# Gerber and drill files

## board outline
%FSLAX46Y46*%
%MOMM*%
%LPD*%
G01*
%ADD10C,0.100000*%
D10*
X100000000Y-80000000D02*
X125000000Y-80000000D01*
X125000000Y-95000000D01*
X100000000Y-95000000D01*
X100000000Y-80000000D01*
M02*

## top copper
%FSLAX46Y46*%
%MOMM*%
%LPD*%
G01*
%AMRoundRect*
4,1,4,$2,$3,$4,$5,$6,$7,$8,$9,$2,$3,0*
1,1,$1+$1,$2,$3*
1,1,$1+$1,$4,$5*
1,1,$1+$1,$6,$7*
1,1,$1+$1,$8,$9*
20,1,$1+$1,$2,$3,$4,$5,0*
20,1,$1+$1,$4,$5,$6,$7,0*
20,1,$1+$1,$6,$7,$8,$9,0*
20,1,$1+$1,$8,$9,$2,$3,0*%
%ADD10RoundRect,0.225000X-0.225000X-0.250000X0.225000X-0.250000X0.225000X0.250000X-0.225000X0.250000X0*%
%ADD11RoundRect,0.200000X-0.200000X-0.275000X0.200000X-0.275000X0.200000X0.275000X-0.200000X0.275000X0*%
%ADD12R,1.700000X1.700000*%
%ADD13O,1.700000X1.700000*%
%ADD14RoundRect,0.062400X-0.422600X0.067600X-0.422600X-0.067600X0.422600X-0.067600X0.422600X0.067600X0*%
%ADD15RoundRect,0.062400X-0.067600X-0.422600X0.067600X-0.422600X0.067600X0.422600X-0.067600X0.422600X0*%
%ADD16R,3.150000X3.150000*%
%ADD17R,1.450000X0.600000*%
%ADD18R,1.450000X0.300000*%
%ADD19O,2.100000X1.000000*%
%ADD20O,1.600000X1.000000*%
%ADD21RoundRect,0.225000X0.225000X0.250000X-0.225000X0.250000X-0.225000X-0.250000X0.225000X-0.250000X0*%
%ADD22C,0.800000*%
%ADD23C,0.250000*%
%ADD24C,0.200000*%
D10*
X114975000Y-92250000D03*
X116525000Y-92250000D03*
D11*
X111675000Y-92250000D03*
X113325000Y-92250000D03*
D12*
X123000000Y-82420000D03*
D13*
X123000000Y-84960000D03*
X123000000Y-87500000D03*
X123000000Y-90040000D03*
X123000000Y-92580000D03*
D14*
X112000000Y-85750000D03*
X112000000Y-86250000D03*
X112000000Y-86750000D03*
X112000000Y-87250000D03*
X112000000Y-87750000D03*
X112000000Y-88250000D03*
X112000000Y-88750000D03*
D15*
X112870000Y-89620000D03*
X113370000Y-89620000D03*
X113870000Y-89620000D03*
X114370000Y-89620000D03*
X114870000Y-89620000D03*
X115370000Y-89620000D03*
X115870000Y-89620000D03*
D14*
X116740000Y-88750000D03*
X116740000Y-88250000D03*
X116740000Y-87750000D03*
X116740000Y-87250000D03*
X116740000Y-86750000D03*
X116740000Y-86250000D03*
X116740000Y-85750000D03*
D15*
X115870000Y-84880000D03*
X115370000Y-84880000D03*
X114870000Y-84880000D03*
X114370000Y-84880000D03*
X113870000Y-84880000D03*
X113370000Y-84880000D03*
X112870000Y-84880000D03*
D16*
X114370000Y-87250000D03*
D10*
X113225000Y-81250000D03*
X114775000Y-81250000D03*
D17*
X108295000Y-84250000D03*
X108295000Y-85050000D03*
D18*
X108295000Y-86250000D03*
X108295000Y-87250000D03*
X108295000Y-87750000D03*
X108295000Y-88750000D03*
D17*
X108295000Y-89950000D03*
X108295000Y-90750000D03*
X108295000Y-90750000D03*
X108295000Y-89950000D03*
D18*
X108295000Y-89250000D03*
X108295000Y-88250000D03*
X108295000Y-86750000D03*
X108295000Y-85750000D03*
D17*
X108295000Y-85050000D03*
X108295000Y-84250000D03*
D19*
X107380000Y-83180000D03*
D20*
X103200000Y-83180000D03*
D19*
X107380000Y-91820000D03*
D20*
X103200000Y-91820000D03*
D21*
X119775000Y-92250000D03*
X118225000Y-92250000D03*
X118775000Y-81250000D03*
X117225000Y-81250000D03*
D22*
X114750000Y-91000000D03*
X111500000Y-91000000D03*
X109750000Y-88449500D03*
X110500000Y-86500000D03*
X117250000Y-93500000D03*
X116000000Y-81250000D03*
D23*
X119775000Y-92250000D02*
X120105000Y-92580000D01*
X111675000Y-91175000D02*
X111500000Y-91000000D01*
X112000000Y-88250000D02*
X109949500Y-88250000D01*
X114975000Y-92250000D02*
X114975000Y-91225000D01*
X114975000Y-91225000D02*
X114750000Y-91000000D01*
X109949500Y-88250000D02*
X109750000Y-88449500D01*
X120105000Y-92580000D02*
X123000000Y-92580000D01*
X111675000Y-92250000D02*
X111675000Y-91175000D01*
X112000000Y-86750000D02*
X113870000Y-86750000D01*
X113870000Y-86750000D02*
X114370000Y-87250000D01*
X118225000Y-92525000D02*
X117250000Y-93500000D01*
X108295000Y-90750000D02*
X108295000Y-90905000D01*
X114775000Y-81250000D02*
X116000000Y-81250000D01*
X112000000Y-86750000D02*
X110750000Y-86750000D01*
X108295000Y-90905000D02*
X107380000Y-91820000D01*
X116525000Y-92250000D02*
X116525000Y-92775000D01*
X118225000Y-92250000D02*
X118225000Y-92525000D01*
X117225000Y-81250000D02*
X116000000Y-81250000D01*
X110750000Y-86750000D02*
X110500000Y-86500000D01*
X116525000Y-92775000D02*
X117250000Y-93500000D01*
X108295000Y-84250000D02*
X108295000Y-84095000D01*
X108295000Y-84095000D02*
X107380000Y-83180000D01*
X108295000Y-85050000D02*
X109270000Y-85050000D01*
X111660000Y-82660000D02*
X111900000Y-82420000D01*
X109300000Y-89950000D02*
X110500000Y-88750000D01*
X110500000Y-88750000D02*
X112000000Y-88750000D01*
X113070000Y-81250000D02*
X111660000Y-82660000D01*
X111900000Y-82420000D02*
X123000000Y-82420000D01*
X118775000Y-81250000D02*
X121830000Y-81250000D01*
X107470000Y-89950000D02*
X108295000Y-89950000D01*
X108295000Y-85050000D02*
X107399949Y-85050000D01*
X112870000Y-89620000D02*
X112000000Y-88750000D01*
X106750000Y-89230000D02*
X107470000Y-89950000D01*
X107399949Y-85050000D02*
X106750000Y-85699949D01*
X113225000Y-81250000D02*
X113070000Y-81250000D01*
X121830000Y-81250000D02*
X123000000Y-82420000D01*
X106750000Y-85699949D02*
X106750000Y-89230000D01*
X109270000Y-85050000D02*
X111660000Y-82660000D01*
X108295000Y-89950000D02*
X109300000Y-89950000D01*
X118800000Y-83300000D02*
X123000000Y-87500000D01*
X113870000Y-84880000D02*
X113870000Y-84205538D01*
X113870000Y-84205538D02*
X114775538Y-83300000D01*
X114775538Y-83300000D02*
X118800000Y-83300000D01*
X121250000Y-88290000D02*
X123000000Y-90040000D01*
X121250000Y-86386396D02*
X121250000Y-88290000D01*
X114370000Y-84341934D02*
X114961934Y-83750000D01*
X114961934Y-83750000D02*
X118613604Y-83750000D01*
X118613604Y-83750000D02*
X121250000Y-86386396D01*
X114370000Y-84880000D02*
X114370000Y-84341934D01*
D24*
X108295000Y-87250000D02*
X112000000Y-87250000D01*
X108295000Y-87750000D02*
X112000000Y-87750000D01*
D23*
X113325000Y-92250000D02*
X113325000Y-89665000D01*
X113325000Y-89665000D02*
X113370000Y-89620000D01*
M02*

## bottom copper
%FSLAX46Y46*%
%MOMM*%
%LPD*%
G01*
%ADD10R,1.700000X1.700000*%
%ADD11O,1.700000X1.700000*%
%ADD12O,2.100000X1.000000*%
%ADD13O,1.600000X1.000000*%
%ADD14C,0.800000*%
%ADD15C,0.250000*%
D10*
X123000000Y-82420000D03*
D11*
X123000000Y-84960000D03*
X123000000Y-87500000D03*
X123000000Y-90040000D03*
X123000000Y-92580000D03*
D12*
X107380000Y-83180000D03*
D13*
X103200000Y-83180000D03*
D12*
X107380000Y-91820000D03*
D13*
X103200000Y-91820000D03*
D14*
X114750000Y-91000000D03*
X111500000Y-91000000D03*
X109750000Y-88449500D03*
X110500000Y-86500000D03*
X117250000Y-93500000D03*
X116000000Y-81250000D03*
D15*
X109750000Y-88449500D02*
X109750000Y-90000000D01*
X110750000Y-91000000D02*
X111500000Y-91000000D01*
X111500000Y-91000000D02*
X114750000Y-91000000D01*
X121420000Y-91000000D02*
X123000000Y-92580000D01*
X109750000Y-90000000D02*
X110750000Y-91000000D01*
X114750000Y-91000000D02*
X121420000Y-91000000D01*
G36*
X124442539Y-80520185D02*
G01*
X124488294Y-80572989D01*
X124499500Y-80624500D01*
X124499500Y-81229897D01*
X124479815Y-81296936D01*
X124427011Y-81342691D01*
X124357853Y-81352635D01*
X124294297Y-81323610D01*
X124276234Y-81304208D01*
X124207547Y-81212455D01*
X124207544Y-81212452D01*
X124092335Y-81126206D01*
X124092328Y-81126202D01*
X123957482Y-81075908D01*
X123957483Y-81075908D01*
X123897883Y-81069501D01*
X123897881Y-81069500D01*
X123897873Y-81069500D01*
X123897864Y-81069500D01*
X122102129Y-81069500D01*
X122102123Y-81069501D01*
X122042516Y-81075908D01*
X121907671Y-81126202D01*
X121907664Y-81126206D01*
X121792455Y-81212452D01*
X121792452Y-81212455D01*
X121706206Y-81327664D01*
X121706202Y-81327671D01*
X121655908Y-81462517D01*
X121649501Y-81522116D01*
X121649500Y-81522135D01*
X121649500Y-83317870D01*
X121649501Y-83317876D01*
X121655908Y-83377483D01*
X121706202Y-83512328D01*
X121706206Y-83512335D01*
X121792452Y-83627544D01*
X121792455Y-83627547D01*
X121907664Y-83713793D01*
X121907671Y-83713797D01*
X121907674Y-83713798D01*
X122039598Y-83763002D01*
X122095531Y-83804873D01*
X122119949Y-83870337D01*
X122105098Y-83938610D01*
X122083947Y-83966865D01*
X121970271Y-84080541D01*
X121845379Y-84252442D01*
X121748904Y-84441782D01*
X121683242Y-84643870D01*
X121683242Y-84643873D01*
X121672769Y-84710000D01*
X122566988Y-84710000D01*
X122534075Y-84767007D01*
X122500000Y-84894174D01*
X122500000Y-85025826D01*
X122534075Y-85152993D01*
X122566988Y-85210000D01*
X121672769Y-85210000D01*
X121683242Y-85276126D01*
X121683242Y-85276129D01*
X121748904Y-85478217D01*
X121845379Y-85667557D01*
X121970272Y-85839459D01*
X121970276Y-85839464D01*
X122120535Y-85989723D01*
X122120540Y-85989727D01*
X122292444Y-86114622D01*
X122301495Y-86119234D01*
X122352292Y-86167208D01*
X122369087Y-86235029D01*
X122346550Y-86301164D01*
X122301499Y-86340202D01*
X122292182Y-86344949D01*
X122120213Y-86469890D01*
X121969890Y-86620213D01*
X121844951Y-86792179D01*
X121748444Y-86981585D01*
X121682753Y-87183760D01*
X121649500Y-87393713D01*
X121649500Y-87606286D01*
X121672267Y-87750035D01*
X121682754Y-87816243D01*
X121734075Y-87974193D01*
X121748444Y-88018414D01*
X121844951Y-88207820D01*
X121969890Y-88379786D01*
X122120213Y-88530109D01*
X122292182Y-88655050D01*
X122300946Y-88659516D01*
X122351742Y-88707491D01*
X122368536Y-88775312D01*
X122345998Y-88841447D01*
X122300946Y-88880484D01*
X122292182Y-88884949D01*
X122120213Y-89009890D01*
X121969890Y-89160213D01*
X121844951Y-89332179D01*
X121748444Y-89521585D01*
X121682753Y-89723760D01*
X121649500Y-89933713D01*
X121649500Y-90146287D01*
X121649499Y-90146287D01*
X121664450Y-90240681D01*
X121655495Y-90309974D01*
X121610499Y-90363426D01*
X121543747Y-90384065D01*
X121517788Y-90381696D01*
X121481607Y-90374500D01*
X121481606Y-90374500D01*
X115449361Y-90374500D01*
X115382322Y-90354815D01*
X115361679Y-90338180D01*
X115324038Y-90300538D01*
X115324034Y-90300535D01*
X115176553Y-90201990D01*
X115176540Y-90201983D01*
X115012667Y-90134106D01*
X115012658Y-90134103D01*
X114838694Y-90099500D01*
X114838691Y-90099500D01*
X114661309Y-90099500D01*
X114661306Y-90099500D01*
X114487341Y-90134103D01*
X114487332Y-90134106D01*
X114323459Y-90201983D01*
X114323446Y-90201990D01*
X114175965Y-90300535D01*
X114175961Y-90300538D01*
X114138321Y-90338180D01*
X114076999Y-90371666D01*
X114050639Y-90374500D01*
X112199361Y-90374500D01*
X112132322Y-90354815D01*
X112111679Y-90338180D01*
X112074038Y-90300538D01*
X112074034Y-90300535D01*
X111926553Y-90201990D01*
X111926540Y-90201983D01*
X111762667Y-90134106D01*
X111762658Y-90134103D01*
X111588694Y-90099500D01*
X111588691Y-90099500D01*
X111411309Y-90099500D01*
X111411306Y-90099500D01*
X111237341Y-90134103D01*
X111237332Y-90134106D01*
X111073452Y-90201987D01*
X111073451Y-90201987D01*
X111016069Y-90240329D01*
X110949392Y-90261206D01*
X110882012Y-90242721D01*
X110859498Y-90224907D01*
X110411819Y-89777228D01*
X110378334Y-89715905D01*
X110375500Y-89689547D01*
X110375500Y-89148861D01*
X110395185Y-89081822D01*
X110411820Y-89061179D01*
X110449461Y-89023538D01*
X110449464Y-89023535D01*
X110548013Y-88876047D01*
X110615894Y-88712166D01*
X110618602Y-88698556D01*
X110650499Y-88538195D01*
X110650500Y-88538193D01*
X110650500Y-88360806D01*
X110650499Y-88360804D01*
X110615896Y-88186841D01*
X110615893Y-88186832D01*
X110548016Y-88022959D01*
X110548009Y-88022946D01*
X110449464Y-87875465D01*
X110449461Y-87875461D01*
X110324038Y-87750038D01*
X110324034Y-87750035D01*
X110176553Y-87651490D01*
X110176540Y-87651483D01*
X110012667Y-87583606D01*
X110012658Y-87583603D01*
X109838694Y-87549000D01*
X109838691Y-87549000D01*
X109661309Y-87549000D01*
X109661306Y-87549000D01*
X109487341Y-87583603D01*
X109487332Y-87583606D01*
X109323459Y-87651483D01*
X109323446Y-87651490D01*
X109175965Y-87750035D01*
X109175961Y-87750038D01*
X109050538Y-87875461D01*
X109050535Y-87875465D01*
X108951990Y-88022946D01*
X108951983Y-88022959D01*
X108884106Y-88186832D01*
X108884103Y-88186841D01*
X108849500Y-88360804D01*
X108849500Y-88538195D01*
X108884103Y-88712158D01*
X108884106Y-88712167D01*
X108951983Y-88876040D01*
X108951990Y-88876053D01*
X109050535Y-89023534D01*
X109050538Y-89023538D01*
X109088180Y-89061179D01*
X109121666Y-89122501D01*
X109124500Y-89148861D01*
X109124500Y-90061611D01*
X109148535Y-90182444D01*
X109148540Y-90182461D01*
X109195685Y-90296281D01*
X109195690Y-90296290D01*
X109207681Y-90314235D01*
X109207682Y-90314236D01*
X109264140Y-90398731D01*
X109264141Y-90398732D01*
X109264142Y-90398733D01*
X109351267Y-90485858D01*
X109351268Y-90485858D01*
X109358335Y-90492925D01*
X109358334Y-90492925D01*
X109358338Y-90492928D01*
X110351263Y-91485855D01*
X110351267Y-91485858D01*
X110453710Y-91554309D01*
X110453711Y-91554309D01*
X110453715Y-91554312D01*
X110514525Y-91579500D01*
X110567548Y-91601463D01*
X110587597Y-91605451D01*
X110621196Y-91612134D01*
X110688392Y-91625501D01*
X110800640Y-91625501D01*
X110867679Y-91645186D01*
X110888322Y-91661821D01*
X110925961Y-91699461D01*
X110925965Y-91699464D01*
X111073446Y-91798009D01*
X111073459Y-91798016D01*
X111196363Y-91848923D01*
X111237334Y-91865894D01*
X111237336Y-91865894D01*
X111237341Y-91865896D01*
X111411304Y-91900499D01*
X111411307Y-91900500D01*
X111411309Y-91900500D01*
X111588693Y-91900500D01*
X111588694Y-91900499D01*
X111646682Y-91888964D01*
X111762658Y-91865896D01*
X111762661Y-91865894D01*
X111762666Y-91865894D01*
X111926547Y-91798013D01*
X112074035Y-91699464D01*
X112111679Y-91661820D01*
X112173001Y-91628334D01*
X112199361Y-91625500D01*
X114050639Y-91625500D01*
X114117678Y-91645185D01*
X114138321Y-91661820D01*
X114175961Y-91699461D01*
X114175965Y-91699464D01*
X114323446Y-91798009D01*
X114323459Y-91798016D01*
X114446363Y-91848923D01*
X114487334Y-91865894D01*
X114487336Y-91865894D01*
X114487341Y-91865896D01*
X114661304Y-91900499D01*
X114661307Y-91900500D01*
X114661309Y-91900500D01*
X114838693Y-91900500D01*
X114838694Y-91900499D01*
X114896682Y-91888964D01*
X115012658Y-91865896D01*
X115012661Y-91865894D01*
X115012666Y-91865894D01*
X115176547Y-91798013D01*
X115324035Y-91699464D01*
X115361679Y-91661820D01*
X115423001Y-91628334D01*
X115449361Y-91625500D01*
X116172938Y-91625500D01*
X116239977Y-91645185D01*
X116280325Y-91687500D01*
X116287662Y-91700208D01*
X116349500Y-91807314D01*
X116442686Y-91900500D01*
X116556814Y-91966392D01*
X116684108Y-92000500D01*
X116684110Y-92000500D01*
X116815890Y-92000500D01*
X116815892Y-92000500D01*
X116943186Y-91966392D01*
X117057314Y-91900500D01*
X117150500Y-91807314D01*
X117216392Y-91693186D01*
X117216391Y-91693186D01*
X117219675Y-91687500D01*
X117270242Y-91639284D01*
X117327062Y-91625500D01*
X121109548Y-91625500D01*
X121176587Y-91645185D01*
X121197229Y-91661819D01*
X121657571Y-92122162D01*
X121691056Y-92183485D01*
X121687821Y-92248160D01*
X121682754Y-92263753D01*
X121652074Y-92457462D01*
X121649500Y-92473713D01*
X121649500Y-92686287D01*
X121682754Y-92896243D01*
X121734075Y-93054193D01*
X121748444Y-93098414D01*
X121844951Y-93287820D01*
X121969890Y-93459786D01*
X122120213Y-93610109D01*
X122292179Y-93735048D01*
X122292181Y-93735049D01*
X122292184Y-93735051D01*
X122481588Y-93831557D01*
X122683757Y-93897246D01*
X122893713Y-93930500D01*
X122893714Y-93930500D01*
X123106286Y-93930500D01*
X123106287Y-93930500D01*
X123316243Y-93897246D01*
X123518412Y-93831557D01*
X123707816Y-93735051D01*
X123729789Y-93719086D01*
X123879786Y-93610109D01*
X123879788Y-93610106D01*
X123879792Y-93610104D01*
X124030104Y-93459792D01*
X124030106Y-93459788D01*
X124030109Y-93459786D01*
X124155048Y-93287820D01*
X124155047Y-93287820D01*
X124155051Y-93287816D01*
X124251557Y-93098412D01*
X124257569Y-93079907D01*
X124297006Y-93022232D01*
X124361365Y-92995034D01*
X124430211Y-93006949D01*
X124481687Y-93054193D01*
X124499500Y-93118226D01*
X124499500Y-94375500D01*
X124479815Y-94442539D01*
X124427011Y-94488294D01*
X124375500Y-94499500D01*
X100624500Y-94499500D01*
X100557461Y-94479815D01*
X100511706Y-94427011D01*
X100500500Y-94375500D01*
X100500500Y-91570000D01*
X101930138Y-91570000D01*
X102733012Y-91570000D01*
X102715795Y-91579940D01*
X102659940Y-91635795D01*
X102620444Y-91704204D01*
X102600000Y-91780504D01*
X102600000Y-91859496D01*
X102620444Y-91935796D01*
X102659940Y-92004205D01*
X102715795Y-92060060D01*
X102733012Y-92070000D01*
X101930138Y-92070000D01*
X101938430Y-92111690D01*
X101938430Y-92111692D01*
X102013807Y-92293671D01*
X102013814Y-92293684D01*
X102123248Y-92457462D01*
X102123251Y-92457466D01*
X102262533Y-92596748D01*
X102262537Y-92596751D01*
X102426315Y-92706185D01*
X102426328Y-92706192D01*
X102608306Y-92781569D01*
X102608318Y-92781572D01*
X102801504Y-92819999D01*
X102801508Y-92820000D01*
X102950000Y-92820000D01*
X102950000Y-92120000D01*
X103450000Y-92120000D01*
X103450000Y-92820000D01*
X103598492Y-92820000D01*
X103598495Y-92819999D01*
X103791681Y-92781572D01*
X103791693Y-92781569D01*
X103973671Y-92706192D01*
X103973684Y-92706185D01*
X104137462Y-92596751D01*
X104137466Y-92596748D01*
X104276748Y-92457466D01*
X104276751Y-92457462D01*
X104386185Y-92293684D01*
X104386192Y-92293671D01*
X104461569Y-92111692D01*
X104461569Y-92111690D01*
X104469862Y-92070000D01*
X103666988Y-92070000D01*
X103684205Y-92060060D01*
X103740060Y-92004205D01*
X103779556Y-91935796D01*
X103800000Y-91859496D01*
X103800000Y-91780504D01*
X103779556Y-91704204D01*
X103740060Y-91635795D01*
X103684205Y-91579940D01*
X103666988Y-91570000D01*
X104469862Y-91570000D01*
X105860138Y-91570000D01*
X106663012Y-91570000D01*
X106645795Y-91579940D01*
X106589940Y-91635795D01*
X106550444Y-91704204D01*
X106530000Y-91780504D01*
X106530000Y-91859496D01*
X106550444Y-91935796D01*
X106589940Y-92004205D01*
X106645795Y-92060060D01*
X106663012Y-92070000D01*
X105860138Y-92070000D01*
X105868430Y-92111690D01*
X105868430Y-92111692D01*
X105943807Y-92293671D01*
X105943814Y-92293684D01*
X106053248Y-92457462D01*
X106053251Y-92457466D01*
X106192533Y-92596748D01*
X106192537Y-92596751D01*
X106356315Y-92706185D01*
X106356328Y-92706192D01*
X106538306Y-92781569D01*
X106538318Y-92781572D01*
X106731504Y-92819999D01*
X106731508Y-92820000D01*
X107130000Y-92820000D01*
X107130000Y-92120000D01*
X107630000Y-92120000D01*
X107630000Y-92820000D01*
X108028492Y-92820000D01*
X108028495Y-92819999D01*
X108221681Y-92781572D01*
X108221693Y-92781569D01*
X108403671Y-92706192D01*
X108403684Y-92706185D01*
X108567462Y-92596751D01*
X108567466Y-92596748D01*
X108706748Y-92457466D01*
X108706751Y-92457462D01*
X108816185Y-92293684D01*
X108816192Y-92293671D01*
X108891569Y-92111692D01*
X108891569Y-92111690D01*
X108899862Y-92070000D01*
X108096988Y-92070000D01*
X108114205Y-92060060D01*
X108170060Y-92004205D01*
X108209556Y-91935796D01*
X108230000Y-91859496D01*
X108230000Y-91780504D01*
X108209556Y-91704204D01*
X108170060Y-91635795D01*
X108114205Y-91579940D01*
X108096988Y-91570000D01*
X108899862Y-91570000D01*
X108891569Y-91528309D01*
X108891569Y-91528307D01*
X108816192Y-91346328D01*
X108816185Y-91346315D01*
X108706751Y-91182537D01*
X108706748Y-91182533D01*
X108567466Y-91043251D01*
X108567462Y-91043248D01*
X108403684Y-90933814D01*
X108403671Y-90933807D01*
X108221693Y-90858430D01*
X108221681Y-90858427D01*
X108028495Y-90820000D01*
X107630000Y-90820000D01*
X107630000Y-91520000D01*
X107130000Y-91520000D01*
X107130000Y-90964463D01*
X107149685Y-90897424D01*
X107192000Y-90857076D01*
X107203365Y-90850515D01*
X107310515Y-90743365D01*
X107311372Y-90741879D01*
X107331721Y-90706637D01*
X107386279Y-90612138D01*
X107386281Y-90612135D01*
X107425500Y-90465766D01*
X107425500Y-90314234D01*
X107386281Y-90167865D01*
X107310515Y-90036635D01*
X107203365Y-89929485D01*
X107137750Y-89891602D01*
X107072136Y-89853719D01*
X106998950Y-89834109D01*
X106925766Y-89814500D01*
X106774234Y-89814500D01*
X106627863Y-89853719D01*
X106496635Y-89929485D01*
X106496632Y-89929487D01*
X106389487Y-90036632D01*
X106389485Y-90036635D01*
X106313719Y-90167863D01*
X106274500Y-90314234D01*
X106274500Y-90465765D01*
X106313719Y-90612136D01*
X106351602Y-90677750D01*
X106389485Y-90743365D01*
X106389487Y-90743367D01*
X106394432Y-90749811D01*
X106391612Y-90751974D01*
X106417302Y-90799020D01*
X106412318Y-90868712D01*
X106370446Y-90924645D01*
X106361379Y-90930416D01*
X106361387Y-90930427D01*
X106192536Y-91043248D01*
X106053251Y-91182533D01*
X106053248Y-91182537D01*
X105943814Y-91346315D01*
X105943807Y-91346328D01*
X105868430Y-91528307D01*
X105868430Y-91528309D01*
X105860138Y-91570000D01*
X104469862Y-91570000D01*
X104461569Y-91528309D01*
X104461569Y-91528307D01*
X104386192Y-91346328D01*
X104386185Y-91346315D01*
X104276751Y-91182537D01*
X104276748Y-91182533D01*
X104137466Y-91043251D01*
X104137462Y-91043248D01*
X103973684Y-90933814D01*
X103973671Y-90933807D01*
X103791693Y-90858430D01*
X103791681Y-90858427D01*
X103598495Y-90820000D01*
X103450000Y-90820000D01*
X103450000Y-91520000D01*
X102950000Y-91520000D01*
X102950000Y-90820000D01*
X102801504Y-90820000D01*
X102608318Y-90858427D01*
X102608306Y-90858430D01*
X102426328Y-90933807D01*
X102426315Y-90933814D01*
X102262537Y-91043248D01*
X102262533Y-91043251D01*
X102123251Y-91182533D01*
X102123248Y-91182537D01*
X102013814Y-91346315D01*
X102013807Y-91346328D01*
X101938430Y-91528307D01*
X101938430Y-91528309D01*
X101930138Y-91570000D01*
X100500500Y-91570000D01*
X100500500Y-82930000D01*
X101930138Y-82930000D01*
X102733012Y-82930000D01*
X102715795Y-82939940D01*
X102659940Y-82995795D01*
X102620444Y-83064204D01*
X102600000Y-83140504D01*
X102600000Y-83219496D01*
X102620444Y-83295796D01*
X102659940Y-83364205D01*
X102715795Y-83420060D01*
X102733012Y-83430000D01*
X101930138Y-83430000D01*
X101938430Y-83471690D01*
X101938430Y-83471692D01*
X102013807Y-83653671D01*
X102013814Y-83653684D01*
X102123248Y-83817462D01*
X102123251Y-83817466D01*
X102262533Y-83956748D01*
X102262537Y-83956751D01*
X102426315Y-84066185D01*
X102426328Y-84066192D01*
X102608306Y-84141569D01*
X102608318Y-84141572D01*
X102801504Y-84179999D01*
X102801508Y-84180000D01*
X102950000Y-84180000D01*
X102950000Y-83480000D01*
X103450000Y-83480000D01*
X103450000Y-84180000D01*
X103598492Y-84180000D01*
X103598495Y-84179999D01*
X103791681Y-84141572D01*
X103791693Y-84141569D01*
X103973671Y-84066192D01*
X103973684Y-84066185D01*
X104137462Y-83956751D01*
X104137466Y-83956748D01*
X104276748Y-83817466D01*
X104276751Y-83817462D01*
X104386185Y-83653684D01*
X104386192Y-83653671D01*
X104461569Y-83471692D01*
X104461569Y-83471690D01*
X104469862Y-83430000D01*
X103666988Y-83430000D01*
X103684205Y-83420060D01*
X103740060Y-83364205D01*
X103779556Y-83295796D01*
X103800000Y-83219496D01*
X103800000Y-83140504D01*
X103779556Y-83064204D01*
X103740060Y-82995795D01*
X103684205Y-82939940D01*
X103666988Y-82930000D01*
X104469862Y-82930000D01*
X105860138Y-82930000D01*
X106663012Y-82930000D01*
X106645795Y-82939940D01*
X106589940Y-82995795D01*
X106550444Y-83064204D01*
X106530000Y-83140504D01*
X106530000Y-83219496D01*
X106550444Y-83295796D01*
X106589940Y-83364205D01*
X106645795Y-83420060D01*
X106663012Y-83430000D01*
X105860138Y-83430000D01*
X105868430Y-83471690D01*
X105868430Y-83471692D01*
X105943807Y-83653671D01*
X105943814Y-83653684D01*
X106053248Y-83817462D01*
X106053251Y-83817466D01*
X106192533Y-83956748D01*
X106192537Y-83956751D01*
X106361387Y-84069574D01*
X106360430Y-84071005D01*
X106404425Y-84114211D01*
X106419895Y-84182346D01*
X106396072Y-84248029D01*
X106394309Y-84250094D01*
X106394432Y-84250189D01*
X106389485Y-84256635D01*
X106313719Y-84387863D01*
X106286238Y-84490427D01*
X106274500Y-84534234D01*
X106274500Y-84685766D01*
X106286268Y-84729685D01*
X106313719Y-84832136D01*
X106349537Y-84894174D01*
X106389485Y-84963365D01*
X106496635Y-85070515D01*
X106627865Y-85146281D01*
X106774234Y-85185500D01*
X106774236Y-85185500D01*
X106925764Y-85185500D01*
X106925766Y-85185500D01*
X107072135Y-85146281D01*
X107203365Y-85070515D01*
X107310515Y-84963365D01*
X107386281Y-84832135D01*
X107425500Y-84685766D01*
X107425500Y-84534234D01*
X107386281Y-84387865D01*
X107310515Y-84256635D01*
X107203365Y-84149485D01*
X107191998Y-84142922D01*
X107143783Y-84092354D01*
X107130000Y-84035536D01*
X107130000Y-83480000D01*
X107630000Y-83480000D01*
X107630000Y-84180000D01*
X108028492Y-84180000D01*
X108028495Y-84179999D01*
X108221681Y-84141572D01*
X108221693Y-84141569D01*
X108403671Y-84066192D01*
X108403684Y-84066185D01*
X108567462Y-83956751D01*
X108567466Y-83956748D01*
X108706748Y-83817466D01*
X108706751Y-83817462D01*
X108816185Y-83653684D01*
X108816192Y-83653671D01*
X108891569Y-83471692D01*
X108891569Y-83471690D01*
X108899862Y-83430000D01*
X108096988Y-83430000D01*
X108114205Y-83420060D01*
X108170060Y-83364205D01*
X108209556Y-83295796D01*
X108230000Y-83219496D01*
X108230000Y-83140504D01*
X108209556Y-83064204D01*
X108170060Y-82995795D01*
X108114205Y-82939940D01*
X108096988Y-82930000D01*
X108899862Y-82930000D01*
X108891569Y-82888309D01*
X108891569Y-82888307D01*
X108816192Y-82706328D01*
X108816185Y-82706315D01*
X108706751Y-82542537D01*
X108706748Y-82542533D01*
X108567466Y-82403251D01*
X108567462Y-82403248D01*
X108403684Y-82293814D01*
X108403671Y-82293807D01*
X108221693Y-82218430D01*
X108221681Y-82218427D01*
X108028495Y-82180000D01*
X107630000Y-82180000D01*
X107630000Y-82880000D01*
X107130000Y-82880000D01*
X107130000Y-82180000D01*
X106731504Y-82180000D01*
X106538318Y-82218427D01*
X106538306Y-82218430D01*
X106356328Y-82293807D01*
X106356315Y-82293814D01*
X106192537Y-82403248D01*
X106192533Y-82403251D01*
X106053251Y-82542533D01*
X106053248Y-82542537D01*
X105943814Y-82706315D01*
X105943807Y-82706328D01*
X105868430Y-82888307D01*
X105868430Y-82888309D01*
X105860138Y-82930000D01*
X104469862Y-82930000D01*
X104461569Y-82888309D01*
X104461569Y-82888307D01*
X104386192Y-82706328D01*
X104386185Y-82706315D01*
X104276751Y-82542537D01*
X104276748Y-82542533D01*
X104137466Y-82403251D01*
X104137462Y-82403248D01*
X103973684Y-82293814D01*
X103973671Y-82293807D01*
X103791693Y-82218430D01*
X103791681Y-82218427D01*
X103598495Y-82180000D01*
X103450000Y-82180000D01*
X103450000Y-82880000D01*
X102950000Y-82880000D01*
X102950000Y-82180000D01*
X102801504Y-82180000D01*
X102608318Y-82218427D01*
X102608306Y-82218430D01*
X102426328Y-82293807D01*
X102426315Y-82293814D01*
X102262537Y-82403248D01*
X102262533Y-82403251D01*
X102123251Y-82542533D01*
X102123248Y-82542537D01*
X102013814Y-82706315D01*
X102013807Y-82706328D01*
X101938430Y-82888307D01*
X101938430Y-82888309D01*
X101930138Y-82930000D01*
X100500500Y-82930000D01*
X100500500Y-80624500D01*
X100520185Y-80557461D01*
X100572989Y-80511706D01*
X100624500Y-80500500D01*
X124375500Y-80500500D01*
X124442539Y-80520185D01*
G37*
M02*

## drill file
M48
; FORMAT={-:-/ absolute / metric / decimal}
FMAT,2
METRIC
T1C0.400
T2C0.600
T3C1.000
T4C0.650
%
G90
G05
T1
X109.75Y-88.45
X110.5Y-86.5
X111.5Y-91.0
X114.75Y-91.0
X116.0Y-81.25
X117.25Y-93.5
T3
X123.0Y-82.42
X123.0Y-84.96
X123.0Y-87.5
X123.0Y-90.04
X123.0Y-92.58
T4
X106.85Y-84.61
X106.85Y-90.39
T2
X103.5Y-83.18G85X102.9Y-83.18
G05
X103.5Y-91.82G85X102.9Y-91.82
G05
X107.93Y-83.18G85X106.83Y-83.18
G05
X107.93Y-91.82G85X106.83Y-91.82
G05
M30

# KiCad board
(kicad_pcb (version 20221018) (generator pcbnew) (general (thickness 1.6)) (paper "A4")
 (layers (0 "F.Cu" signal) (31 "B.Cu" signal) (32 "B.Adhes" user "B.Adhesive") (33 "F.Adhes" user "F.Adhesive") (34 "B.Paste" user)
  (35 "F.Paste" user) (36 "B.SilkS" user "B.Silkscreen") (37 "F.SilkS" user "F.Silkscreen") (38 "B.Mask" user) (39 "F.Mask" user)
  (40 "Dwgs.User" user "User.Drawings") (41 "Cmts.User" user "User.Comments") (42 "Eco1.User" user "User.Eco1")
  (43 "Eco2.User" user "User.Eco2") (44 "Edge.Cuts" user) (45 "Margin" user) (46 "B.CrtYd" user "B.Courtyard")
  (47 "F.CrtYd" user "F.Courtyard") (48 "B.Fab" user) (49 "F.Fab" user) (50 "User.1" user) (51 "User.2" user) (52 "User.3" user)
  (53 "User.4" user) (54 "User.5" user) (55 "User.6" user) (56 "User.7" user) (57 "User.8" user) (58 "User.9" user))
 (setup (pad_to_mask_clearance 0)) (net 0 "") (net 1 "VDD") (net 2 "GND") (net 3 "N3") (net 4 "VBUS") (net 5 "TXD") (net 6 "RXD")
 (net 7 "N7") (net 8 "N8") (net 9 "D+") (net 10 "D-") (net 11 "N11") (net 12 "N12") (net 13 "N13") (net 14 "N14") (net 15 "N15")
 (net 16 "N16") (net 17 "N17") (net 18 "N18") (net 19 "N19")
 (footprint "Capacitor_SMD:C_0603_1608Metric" (layer "F.Cu") (at 115.75 92.25)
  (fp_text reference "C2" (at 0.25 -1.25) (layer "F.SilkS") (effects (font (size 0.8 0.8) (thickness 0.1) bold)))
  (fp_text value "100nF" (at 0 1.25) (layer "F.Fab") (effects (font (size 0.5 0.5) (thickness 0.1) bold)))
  (pad "1" smd roundrect (at -0.775 0) (size 0.9 0.95) (layers "F.Cu" "F.Paste" "F.Mask") (roundrect_rratio 0.25) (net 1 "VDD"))
  (pad "2" smd roundrect (at 0.775 0) (size 0.9 0.95) (layers "F.Cu" "F.Paste" "F.Mask") (roundrect_rratio 0.25) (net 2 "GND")))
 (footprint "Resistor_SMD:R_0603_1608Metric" (layer "F.Cu") (at 112.5 92.25)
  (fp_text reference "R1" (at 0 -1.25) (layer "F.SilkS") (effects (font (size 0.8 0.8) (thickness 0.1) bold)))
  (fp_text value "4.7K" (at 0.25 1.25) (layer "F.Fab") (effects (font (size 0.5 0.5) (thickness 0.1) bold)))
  (pad "1" smd roundrect (at -0.825 0) (size 0.8 0.95) (layers "F.Cu" "F.Paste" "F.Mask") (roundrect_rratio 0.25) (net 1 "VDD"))
  (pad "2" smd roundrect (at 0.825 0) (size 0.8 0.95) (layers "F.Cu" "F.Paste" "F.Mask") (roundrect_rratio 0.25) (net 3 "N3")))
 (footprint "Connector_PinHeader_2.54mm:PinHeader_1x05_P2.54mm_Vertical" (layer "F.Cu") (at 123 82.42)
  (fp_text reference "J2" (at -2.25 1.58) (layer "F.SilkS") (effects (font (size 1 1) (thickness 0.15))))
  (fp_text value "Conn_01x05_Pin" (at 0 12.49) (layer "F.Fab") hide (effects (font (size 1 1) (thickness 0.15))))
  (pad "1" thru_hole rect (at 0 0) (size 1.7 1.7) (drill 1) (layers "*.Cu" "*.Mask") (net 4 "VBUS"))
  (pad "2" thru_hole oval (at 0 2.54) (size 1.7 1.7) (drill 1) (layers "*.Cu" "*.Mask") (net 2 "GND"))
  (pad "3" thru_hole oval (at 0 5.08) (size 1.7 1.7) (drill 1) (layers "*.Cu" "*.Mask") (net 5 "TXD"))
  (pad "4" thru_hole oval (at 0 7.62) (size 1.7 1.7) (drill 1) (layers "*.Cu" "*.Mask") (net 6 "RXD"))
  (pad "5" thru_hole oval (at 0 10.16) (size 1.7 1.7) (drill 1) (layers "*.Cu" "*.Mask") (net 1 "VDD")))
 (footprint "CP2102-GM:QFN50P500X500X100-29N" (layer "F.Cu") (at 114.37 87.25)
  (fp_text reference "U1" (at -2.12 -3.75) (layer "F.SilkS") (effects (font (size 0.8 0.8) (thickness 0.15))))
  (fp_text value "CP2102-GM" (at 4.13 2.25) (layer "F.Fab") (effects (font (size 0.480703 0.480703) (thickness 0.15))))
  (pad "1" smd roundrect (at -2.37 -1.5 270) (size 0.26 0.97) (layers "F.Cu" "F.Paste" "F.Mask") (roundrect_rratio 0.24) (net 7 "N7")
   (solder_mask_margin 0.102))
  (pad "2" smd roundrect (at -2.37 -1 270) (size 0.26 0.97) (layers "F.Cu" "F.Paste" "F.Mask") (roundrect_rratio 0.24) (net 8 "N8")
   (solder_mask_margin 0.102))
  (pad "3" smd roundrect (at -2.37 -0.5 270) (size 0.26 0.97) (layers "F.Cu" "F.Paste" "F.Mask") (roundrect_rratio 0.24) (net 2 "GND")
   (solder_mask_margin 0.102))
  (pad "4" smd roundrect (at -2.37 0 270) (size 0.26 0.97) (layers "F.Cu" "F.Paste" "F.Mask") (roundrect_rratio 0.24) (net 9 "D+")
   (solder_mask_margin 0.102))
  (pad "5" smd roundrect (at -2.37 0.5 270) (size 0.26 0.97) (layers "F.Cu" "F.Paste" "F.Mask") (roundrect_rratio 0.24) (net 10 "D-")
   (solder_mask_margin 0.102))
  (pad "6" smd roundrect (at -2.37 1 270) (size 0.26 0.97) (layers "F.Cu" "F.Paste" "F.Mask") (roundrect_rratio 0.24) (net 1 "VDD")
   (solder_mask_margin 0.102))
  (pad "7" smd roundrect (at -2.37 1.5 270) (size 0.26 0.97) (layers "F.Cu" "F.Paste" "F.Mask") (roundrect_rratio 0.24) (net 4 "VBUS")
   (solder_mask_margin 0.102))
  (pad "8" smd roundrect (at -1.5 2.37) (size 0.26 0.97) (layers "F.Cu" "F.Paste" "F.Mask") (roundrect_rratio 0.24) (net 4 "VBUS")
   (solder_mask_margin 0.102))
  (pad "9" smd roundrect (at -1 2.37) (size 0.26 0.97) (layers "F.Cu" "F.Paste" "F.Mask") (roundrect_rratio 0.24) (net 3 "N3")
   (solder_mask_margin 0.102))
  (pad "10" smd roundrect (at -0.5 2.37) (size 0.26 0.97) (layers "F.Cu" "F.Paste" "F.Mask") (roundrect_rratio 0.24)
   (solder_mask_margin 0.102))
  (pad "11" smd roundrect (at 0 2.37) (size 0.26 0.97) (layers "F.Cu" "F.Paste" "F.Mask") (roundrect_rratio 0.24) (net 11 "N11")
   (solder_mask_margin 0.102))
  (pad "12" smd roundrect (at 0.5 2.37) (size 0.26 0.97) (layers "F.Cu" "F.Paste" "F.Mask") (roundrect_rratio 0.24) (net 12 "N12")
   (solder_mask_margin 0.102))
  (pad "13" smd roundrect (at 1 2.37) (size 0.26 0.97) (layers "F.Cu" "F.Paste" "F.Mask") (roundrect_rratio 0.24) (solder_mask_margin 0.102))
  (pad "14" smd roundrect (at 1.5 2.37) (size 0.26 0.97) (layers "F.Cu" "F.Paste" "F.Mask") (roundrect_rratio 0.24)
   (solder_mask_margin 0.102))
  (pad "15" smd roundrect (at 2.37 1.5 270) (size 0.26 0.97) (layers "F.Cu" "F.Paste" "F.Mask") (roundrect_rratio 0.24)
   (solder_mask_margin 0.102))
  (pad "16" smd roundrect (at 2.37 1 270) (size 0.26 0.97) (layers "F.Cu" "F.Paste" "F.Mask") (roundrect_rratio 0.24)
   (solder_mask_margin 0.102))
  (pad "17" smd roundrect (at 2.37 0.5 270) (size 0.26 0.97) (layers "F.Cu" "F.Paste" "F.Mask") (roundrect_rratio 0.24)
   (solder_mask_margin 0.102))
  (pad "18" smd roundrect (at 2.37 0 270) (size 0.26 0.97) (layers "F.Cu" "F.Paste" "F.Mask") (roundrect_rratio 0.24) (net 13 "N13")
   (solder_mask_margin 0.102))
  (pad "19" smd roundrect (at 2.37 -0.5 270) (size 0.26 0.97) (layers "F.Cu" "F.Paste" "F.Mask") (roundrect_rratio 0.24)
   (solder_mask_margin 0.102))
  (pad "20" smd roundrect (at 2.37 -1 270) (size 0.26 0.97) (layers "F.Cu" "F.Paste" "F.Mask") (roundrect_rratio 0.24)
   (solder_mask_margin 0.102))
  (pad "21" smd roundrect (at 2.37 -1.5 270) (size 0.26 0.97) (layers "F.Cu" "F.Paste" "F.Mask") (roundrect_rratio 0.24)
   (solder_mask_margin 0.102))
  (pad "22" smd roundrect (at 1.5 -2.37) (size 0.26 0.97) (layers "F.Cu" "F.Paste" "F.Mask") (roundrect_rratio 0.24)
   (solder_mask_margin 0.102))
  (pad "23" smd roundrect (at 1 -2.37) (size 0.26 0.97) (layers "F.Cu" "F.Paste" "F.Mask") (roundrect_rratio 0.24) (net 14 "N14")
   (solder_mask_margin 0.102))
  (pad "24" smd roundrect (at 0.5 -2.37) (size 0.26 0.97) (layers "F.Cu" "F.Paste" "F.Mask") (roundrect_rratio 0.24) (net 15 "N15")
   (solder_mask_margin 0.102))
  (pad "25" smd roundrect (at 0 -2.37) (size 0.26 0.97) (layers "F.Cu" "F.Paste" "F.Mask") (roundrect_rratio 0.24) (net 6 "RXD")
   (solder_mask_margin 0.102))
  (pad "26" smd roundrect (at -0.5 -2.37) (size 0.26 0.97) (layers "F.Cu" "F.Paste" "F.Mask") (roundrect_rratio 0.24) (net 5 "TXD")
   (solder_mask_margin 0.102))
  (pad "27" smd roundrect (at -1 -2.37) (size 0.26 0.97) (layers "F.Cu" "F.Paste" "F.Mask") (roundrect_rratio 0.24) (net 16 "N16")
   (solder_mask_margin 0.102))
  (pad "28" smd roundrect (at -1.5 -2.37) (size 0.26 0.97) (layers "F.Cu" "F.Paste" "F.Mask") (roundrect_rratio 0.24) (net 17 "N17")
   (solder_mask_margin 0.102))
  (pad "29" smd rect (at 0 0) (size 3.15 3.15) (layers "F.Cu" "F.Mask") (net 2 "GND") (solder_mask_margin 0.102)))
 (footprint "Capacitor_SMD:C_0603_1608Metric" (layer "F.Cu") (at 114 81.25)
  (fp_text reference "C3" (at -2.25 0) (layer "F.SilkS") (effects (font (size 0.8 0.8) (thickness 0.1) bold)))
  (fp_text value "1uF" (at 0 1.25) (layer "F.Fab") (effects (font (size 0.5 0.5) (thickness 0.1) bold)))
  (pad "1" smd roundrect (at -0.775 0) (size 0.9 0.95) (layers "F.Cu" "F.Paste" "F.Mask") (roundrect_rratio 0.25) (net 4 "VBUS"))
  (pad "2" smd roundrect (at 0.775 0) (size 0.9 0.95) (layers "F.Cu" "F.Paste" "F.Mask") (roundrect_rratio 0.25) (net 2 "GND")))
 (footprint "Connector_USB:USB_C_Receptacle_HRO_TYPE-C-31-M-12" (layer "F.Cu") (at 104.25 87.5 -90)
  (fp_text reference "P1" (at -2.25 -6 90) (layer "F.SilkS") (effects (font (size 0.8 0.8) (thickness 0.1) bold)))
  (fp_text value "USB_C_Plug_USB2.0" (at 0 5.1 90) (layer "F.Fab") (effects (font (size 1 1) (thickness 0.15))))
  (pad "" np_thru_hole circle (at -2.89 -2.6 270) (size 0.65 0.65) (drill 0.65) (layers "*.Cu" "*.Mask"))
  (pad "" np_thru_hole circle (at 2.89 -2.6 270) (size 0.65 0.65) (drill 0.65) (layers "*.Cu" "*.Mask"))
  (pad "A1" smd rect (at -3.25 -4.045 270) (size 0.6 1.45) (layers "F.Cu" "F.Paste" "F.Mask") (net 2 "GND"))
  (pad "A4" smd rect (at -2.45 -4.045 270) (size 0.6 1.45) (layers "F.Cu" "F.Paste" "F.Mask") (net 4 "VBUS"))
  (pad "A5" smd rect (at -1.25 -4.045 270) (size 0.3 1.45) (layers "F.Cu" "F.Paste" "F.Mask") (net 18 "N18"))
  (pad "A6" smd rect (at -0.25 -4.045 270) (size 0.3 1.45) (layers "F.Cu" "F.Paste" "F.Mask") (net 9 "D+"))
  (pad "A7" smd rect (at 0.25 -4.045 270) (size 0.3 1.45) (layers "F.Cu" "F.Paste" "F.Mask") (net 10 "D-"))
  (pad "A8" smd rect (at 1.25 -4.045 270) (size 0.3 1.45) (layers "F.Cu" "F.Paste" "F.Mask"))
  (pad "A9" smd rect (at 2.45 -4.045 270) (size 0.6 1.45) (layers "F.Cu" "F.Paste" "F.Mask") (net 4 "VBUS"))
  (pad "A12" smd rect (at 3.25 -4.045 270) (size 0.6 1.45) (layers "F.Cu" "F.Paste" "F.Mask") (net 2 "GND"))
  (pad "B1" smd rect (at 3.25 -4.045 270) (size 0.6 1.45) (layers "F.Cu" "F.Paste" "F.Mask") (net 2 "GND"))
  (pad "B4" smd rect (at 2.45 -4.045 270) (size 0.6 1.45) (layers "F.Cu" "F.Paste" "F.Mask") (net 4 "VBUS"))
  (pad "B5" smd rect (at 1.75 -4.045 270) (size 0.3 1.45) (layers "F.Cu" "F.Paste" "F.Mask") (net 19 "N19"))
  (pad "B6" smd rect (at 0.75 -4.045 270) (size 0.3 1.45) (layers "F.Cu" "F.Paste" "F.Mask"))
  (pad "B7" smd rect (at -0.75 -4.045 270) (size 0.3 1.45) (layers "F.Cu" "F.Paste" "F.Mask"))
  (pad "B8" smd rect (at -1.75 -4.045 270) (size 0.3 1.45) (layers "F.Cu" "F.Paste" "F.Mask"))
  (pad "B9" smd rect (at -2.45 -4.045 270) (size 0.6 1.45) (layers "F.Cu" "F.Paste" "F.Mask") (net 4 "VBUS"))
  (pad "B12" smd rect (at -3.25 -4.045 270) (size 0.6 1.45) (layers "F.Cu" "F.Paste" "F.Mask") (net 2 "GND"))
  (pad "S1" thru_hole oval (at -4.32 -3.13 270) (size 1 2.1) (drill oval 0.6 1.7) (layers "*.Cu" "*.Mask") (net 2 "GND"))
  (pad "S1" thru_hole oval (at -4.32 1.05 270) (size 1 1.6) (drill oval 0.6 1.2) (layers "*.Cu" "*.Mask") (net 2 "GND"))
  (pad "S1" thru_hole oval (at 4.32 -3.13 270) (size 1 2.1) (drill oval 0.6 1.7) (layers "*.Cu" "*.Mask") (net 2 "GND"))
  (pad "S1" thru_hole oval (at 4.32 1.05 270) (size 1 1.6) (drill oval 0.6 1.2) (layers "*.Cu" "*.Mask") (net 2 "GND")))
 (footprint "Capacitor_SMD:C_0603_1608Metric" (layer "F.Cu") (at 119 92.25 180)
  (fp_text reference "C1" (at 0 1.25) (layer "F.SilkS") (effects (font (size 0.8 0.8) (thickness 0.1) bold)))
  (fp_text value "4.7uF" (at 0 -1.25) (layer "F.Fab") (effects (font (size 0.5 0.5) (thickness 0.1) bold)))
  (pad "1" smd roundrect (at -0.775 0 180) (size 0.9 0.95) (layers "F.Cu" "F.Paste" "F.Mask") (roundrect_rratio 0.25) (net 1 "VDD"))
  (pad "2" smd roundrect (at 0.775 0 180) (size 0.9 0.95) (layers "F.Cu" "F.Paste" "F.Mask") (roundrect_rratio 0.25) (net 2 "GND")))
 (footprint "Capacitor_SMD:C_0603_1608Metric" (layer "F.Cu") (at 118 81.25 180)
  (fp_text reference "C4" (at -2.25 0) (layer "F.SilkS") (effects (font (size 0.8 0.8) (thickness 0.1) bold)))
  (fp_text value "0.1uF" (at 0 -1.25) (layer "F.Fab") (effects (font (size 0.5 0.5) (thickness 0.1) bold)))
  (pad "1" smd roundrect (at -0.775 0 180) (size 0.9 0.95) (layers "F.Cu" "F.Paste" "F.Mask") (roundrect_rratio 0.25) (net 4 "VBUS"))
  (pad "2" smd roundrect (at 0.775 0 180) (size 0.9 0.95) (layers "F.Cu" "F.Paste" "F.Mask") (roundrect_rratio 0.25) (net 2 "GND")))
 (gr_rect (start 100 80) (end 125 95) (stroke (width 0.1) (type default)) (fill none) (layer "Edge.Cuts"))
 (gr_rect (start 116.75 91.5) (end 116.75 91.5) (stroke (width 0.1) (type default)) (fill none) (layer "Edge.Cuts"))
 (segment (start 119.775 92.25) (end 120.105 92.58) (width 0.25) (layer "F.Cu") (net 1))
 (segment (start 111.675 91.175) (end 111.5 91) (width 0.25) (layer "F.Cu") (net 1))
 (segment (start 112 88.25) (end 109.9495 88.25) (width 0.25) (layer "F.Cu") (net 1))
 (segment (start 114.975 92.25) (end 114.975 91.225) (width 0.25) (layer "F.Cu") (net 1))
 (segment (start 114.975 91.225) (end 114.75 91) (width 0.25) (layer "F.Cu") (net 1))
 (segment (start 109.9495 88.25) (end 109.75 88.4495) (width 0.25) (layer "F.Cu") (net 1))
 (segment (start 120.105 92.58) (end 123 92.58) (width 0.25) (layer "F.Cu") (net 1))
 (segment (start 111.675 92.25) (end 111.675 91.175) (width 0.25) (layer "F.Cu") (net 1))
 (via (at 114.75 91) (size 0.8) (drill 0.4) (layers "F.Cu" "B.Cu") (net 1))
 (via (at 111.5 91) (size 0.8) (drill 0.4) (layers "F.Cu" "B.Cu") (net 1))
 (via (at 109.75 88.4495) (size 0.8) (drill 0.4) (layers "F.Cu" "B.Cu") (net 1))
 (segment (start 109.75 88.4495) (end 109.75 90) (width 0.25) (layer "B.Cu") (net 1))
 (segment (start 110.75 91) (end 111.5 91) (width 0.25) (layer "B.Cu") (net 1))
 (segment (start 111.5 91) (end 114.75 91) (width 0.25) (layer "B.Cu") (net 1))
 (segment (start 121.42 91) (end 123 92.58) (width 0.25) (layer "B.Cu") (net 1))
 (segment (start 109.75 90) (end 110.75 91) (width 0.25) (layer "B.Cu") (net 1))
 (segment (start 114.75 91) (end 121.42 91) (width 0.25) (layer "B.Cu") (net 1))
 (segment (start 112 86.75) (end 113.87 86.75) (width 0.25) (layer "F.Cu") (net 2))
 (segment (start 113.87 86.75) (end 114.37 87.25) (width 0.25) (layer "F.Cu") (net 2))
 (segment (start 118.225 92.525) (end 117.25 93.5) (width 0.25) (layer "F.Cu") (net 2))
 (segment (start 108.295 90.75) (end 108.295 90.905) (width 0.25) (layer "F.Cu") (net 2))
 (segment (start 114.775 81.25) (end 116 81.25) (width 0.25) (layer "F.Cu") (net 2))
 (segment (start 112 86.75) (end 110.75 86.75) (width 0.25) (layer "F.Cu") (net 2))
 (segment (start 108.295 90.905) (end 107.38 91.82) (width 0.25) (layer "F.Cu") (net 2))
 (segment (start 116.525 92.25) (end 116.525 92.775) (width 0.25) (layer "F.Cu") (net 2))
 (segment (start 118.225 92.25) (end 118.225 92.525) (width 0.25) (layer "F.Cu") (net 2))
 (segment (start 117.225 81.25) (end 116 81.25) (width 0.25) (layer "F.Cu") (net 2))
 (segment (start 110.75 86.75) (end 110.5 86.5) (width 0.25) (layer "F.Cu") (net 2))
 (segment (start 116.525 92.775) (end 117.25 93.5) (width 0.25) (layer "F.Cu") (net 2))
 (segment (start 108.295 84.25) (end 108.295 84.095) (width 0.25) (layer "F.Cu") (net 2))
 (segment (start 108.295 84.095) (end 107.38 83.18) (width 0.25) (layer "F.Cu") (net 2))
 (via (at 110.5 86.5) (size 0.8) (drill 0.4) (layers "F.Cu" "B.Cu") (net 2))
 (via (at 117.25 93.5) (size 0.8) (drill 0.4) (layers "F.Cu" "B.Cu") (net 2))
 (via (at 116 81.25) (size 0.8) (drill 0.4) (layers "F.Cu" "B.Cu") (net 2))
 (segment (start 108.295 85.05) (end 109.27 85.05) (width 0.25) (layer "F.Cu") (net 4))
 (segment (start 111.66 82.66) (end 111.9 82.42) (width 0.25) (layer "F.Cu") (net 4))
 (segment (start 109.3 89.95) (end 110.5 88.75) (width 0.25) (layer "F.Cu") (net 4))
 (segment (start 110.5 88.75) (end 112 88.75) (width 0.25) (layer "F.Cu") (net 4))
 (segment (start 113.07 81.25) (end 111.66 82.66) (width 0.25) (layer "F.Cu") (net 4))
 (segment (start 111.9 82.42) (end 123 82.42) (width 0.25) (layer "F.Cu") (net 4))
 (segment (start 118.775 81.25) (end 121.83 81.25) (width 0.25) (layer "F.Cu") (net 4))
 (segment (start 107.47 89.95) (end 108.295 89.95) (width 0.25) (layer "F.Cu") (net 4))
 (segment (start 108.295 85.05) (end 107.399949 85.05) (width 0.25) (layer "F.Cu") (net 4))
 (segment (start 112.87 89.62) (end 112 88.75) (width 0.25) (layer "F.Cu") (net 4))
 (segment (start 106.75 89.23) (end 107.47 89.95) (width 0.25) (layer "F.Cu") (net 4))
 (segment (start 107.399949 85.05) (end 106.75 85.699949) (width 0.25) (layer "F.Cu") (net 4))
 (segment (start 113.225 81.25) (end 113.07 81.25) (width 0.25) (layer "F.Cu") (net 4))
 (segment (start 121.83 81.25) (end 123 82.42) (width 0.25) (layer "F.Cu") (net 4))
 (segment (start 106.75 85.699949) (end 106.75 89.23) (width 0.25) (layer "F.Cu") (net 4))
 (segment (start 109.27 85.05) (end 111.66 82.66) (width 0.25) (layer "F.Cu") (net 4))
 (segment (start 108.295 89.95) (end 109.3 89.95) (width 0.25) (layer "F.Cu") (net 4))
 (segment (start 118.8 83.3) (end 123 87.5) (width 0.25) (layer "F.Cu") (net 5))
 (segment (start 113.87 84.88) (end 113.87 84.205538) (width 0.25) (layer "F.Cu") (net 5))
 (segment (start 113.87 84.205538) (end 114.775538 83.3) (width 0.25) (layer "F.Cu") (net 5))
 (segment (start 114.775538 83.3) (end 118.8 83.3) (width 0.25) (layer "F.Cu") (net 5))
 (segment (start 121.25 88.29) (end 123 90.04) (width 0.25) (layer "F.Cu") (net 6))
 (segment (start 121.25 86.386396) (end 121.25 88.29) (width 0.25) (layer "F.Cu") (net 6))
 (segment (start 114.37 84.341934) (end 114.961934 83.75) (width 0.25) (layer "F.Cu") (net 6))
 (segment (start 114.961934 83.75) (end 118.613604 83.75) (width 0.25) (layer "F.Cu") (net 6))
 (segment (start 118.613604 83.75) (end 121.25 86.386396) (width 0.25) (layer "F.Cu") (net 6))
 (segment (start 114.37 84.88) (end 114.37 84.341934) (width 0.25) (layer "F.Cu") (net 6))
 (segment (start 108.295 87.25) (end 112 87.25) (width 0.2) (layer "F.Cu") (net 9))
 (segment (start 108.295 87.75) (end 112 87.75) (width 0.2) (layer "F.Cu") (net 10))
 (segment (start 113.325 92.25) (end 113.325 89.665) (width 0.25) (layer "F.Cu") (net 3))
 (segment (start 113.325 89.665) (end 113.37 89.62) (width 0.25) (layer "F.Cu") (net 3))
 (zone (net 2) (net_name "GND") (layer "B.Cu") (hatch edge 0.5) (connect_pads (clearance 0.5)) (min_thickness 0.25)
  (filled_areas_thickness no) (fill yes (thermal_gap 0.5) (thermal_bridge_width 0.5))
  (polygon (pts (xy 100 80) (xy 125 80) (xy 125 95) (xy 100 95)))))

